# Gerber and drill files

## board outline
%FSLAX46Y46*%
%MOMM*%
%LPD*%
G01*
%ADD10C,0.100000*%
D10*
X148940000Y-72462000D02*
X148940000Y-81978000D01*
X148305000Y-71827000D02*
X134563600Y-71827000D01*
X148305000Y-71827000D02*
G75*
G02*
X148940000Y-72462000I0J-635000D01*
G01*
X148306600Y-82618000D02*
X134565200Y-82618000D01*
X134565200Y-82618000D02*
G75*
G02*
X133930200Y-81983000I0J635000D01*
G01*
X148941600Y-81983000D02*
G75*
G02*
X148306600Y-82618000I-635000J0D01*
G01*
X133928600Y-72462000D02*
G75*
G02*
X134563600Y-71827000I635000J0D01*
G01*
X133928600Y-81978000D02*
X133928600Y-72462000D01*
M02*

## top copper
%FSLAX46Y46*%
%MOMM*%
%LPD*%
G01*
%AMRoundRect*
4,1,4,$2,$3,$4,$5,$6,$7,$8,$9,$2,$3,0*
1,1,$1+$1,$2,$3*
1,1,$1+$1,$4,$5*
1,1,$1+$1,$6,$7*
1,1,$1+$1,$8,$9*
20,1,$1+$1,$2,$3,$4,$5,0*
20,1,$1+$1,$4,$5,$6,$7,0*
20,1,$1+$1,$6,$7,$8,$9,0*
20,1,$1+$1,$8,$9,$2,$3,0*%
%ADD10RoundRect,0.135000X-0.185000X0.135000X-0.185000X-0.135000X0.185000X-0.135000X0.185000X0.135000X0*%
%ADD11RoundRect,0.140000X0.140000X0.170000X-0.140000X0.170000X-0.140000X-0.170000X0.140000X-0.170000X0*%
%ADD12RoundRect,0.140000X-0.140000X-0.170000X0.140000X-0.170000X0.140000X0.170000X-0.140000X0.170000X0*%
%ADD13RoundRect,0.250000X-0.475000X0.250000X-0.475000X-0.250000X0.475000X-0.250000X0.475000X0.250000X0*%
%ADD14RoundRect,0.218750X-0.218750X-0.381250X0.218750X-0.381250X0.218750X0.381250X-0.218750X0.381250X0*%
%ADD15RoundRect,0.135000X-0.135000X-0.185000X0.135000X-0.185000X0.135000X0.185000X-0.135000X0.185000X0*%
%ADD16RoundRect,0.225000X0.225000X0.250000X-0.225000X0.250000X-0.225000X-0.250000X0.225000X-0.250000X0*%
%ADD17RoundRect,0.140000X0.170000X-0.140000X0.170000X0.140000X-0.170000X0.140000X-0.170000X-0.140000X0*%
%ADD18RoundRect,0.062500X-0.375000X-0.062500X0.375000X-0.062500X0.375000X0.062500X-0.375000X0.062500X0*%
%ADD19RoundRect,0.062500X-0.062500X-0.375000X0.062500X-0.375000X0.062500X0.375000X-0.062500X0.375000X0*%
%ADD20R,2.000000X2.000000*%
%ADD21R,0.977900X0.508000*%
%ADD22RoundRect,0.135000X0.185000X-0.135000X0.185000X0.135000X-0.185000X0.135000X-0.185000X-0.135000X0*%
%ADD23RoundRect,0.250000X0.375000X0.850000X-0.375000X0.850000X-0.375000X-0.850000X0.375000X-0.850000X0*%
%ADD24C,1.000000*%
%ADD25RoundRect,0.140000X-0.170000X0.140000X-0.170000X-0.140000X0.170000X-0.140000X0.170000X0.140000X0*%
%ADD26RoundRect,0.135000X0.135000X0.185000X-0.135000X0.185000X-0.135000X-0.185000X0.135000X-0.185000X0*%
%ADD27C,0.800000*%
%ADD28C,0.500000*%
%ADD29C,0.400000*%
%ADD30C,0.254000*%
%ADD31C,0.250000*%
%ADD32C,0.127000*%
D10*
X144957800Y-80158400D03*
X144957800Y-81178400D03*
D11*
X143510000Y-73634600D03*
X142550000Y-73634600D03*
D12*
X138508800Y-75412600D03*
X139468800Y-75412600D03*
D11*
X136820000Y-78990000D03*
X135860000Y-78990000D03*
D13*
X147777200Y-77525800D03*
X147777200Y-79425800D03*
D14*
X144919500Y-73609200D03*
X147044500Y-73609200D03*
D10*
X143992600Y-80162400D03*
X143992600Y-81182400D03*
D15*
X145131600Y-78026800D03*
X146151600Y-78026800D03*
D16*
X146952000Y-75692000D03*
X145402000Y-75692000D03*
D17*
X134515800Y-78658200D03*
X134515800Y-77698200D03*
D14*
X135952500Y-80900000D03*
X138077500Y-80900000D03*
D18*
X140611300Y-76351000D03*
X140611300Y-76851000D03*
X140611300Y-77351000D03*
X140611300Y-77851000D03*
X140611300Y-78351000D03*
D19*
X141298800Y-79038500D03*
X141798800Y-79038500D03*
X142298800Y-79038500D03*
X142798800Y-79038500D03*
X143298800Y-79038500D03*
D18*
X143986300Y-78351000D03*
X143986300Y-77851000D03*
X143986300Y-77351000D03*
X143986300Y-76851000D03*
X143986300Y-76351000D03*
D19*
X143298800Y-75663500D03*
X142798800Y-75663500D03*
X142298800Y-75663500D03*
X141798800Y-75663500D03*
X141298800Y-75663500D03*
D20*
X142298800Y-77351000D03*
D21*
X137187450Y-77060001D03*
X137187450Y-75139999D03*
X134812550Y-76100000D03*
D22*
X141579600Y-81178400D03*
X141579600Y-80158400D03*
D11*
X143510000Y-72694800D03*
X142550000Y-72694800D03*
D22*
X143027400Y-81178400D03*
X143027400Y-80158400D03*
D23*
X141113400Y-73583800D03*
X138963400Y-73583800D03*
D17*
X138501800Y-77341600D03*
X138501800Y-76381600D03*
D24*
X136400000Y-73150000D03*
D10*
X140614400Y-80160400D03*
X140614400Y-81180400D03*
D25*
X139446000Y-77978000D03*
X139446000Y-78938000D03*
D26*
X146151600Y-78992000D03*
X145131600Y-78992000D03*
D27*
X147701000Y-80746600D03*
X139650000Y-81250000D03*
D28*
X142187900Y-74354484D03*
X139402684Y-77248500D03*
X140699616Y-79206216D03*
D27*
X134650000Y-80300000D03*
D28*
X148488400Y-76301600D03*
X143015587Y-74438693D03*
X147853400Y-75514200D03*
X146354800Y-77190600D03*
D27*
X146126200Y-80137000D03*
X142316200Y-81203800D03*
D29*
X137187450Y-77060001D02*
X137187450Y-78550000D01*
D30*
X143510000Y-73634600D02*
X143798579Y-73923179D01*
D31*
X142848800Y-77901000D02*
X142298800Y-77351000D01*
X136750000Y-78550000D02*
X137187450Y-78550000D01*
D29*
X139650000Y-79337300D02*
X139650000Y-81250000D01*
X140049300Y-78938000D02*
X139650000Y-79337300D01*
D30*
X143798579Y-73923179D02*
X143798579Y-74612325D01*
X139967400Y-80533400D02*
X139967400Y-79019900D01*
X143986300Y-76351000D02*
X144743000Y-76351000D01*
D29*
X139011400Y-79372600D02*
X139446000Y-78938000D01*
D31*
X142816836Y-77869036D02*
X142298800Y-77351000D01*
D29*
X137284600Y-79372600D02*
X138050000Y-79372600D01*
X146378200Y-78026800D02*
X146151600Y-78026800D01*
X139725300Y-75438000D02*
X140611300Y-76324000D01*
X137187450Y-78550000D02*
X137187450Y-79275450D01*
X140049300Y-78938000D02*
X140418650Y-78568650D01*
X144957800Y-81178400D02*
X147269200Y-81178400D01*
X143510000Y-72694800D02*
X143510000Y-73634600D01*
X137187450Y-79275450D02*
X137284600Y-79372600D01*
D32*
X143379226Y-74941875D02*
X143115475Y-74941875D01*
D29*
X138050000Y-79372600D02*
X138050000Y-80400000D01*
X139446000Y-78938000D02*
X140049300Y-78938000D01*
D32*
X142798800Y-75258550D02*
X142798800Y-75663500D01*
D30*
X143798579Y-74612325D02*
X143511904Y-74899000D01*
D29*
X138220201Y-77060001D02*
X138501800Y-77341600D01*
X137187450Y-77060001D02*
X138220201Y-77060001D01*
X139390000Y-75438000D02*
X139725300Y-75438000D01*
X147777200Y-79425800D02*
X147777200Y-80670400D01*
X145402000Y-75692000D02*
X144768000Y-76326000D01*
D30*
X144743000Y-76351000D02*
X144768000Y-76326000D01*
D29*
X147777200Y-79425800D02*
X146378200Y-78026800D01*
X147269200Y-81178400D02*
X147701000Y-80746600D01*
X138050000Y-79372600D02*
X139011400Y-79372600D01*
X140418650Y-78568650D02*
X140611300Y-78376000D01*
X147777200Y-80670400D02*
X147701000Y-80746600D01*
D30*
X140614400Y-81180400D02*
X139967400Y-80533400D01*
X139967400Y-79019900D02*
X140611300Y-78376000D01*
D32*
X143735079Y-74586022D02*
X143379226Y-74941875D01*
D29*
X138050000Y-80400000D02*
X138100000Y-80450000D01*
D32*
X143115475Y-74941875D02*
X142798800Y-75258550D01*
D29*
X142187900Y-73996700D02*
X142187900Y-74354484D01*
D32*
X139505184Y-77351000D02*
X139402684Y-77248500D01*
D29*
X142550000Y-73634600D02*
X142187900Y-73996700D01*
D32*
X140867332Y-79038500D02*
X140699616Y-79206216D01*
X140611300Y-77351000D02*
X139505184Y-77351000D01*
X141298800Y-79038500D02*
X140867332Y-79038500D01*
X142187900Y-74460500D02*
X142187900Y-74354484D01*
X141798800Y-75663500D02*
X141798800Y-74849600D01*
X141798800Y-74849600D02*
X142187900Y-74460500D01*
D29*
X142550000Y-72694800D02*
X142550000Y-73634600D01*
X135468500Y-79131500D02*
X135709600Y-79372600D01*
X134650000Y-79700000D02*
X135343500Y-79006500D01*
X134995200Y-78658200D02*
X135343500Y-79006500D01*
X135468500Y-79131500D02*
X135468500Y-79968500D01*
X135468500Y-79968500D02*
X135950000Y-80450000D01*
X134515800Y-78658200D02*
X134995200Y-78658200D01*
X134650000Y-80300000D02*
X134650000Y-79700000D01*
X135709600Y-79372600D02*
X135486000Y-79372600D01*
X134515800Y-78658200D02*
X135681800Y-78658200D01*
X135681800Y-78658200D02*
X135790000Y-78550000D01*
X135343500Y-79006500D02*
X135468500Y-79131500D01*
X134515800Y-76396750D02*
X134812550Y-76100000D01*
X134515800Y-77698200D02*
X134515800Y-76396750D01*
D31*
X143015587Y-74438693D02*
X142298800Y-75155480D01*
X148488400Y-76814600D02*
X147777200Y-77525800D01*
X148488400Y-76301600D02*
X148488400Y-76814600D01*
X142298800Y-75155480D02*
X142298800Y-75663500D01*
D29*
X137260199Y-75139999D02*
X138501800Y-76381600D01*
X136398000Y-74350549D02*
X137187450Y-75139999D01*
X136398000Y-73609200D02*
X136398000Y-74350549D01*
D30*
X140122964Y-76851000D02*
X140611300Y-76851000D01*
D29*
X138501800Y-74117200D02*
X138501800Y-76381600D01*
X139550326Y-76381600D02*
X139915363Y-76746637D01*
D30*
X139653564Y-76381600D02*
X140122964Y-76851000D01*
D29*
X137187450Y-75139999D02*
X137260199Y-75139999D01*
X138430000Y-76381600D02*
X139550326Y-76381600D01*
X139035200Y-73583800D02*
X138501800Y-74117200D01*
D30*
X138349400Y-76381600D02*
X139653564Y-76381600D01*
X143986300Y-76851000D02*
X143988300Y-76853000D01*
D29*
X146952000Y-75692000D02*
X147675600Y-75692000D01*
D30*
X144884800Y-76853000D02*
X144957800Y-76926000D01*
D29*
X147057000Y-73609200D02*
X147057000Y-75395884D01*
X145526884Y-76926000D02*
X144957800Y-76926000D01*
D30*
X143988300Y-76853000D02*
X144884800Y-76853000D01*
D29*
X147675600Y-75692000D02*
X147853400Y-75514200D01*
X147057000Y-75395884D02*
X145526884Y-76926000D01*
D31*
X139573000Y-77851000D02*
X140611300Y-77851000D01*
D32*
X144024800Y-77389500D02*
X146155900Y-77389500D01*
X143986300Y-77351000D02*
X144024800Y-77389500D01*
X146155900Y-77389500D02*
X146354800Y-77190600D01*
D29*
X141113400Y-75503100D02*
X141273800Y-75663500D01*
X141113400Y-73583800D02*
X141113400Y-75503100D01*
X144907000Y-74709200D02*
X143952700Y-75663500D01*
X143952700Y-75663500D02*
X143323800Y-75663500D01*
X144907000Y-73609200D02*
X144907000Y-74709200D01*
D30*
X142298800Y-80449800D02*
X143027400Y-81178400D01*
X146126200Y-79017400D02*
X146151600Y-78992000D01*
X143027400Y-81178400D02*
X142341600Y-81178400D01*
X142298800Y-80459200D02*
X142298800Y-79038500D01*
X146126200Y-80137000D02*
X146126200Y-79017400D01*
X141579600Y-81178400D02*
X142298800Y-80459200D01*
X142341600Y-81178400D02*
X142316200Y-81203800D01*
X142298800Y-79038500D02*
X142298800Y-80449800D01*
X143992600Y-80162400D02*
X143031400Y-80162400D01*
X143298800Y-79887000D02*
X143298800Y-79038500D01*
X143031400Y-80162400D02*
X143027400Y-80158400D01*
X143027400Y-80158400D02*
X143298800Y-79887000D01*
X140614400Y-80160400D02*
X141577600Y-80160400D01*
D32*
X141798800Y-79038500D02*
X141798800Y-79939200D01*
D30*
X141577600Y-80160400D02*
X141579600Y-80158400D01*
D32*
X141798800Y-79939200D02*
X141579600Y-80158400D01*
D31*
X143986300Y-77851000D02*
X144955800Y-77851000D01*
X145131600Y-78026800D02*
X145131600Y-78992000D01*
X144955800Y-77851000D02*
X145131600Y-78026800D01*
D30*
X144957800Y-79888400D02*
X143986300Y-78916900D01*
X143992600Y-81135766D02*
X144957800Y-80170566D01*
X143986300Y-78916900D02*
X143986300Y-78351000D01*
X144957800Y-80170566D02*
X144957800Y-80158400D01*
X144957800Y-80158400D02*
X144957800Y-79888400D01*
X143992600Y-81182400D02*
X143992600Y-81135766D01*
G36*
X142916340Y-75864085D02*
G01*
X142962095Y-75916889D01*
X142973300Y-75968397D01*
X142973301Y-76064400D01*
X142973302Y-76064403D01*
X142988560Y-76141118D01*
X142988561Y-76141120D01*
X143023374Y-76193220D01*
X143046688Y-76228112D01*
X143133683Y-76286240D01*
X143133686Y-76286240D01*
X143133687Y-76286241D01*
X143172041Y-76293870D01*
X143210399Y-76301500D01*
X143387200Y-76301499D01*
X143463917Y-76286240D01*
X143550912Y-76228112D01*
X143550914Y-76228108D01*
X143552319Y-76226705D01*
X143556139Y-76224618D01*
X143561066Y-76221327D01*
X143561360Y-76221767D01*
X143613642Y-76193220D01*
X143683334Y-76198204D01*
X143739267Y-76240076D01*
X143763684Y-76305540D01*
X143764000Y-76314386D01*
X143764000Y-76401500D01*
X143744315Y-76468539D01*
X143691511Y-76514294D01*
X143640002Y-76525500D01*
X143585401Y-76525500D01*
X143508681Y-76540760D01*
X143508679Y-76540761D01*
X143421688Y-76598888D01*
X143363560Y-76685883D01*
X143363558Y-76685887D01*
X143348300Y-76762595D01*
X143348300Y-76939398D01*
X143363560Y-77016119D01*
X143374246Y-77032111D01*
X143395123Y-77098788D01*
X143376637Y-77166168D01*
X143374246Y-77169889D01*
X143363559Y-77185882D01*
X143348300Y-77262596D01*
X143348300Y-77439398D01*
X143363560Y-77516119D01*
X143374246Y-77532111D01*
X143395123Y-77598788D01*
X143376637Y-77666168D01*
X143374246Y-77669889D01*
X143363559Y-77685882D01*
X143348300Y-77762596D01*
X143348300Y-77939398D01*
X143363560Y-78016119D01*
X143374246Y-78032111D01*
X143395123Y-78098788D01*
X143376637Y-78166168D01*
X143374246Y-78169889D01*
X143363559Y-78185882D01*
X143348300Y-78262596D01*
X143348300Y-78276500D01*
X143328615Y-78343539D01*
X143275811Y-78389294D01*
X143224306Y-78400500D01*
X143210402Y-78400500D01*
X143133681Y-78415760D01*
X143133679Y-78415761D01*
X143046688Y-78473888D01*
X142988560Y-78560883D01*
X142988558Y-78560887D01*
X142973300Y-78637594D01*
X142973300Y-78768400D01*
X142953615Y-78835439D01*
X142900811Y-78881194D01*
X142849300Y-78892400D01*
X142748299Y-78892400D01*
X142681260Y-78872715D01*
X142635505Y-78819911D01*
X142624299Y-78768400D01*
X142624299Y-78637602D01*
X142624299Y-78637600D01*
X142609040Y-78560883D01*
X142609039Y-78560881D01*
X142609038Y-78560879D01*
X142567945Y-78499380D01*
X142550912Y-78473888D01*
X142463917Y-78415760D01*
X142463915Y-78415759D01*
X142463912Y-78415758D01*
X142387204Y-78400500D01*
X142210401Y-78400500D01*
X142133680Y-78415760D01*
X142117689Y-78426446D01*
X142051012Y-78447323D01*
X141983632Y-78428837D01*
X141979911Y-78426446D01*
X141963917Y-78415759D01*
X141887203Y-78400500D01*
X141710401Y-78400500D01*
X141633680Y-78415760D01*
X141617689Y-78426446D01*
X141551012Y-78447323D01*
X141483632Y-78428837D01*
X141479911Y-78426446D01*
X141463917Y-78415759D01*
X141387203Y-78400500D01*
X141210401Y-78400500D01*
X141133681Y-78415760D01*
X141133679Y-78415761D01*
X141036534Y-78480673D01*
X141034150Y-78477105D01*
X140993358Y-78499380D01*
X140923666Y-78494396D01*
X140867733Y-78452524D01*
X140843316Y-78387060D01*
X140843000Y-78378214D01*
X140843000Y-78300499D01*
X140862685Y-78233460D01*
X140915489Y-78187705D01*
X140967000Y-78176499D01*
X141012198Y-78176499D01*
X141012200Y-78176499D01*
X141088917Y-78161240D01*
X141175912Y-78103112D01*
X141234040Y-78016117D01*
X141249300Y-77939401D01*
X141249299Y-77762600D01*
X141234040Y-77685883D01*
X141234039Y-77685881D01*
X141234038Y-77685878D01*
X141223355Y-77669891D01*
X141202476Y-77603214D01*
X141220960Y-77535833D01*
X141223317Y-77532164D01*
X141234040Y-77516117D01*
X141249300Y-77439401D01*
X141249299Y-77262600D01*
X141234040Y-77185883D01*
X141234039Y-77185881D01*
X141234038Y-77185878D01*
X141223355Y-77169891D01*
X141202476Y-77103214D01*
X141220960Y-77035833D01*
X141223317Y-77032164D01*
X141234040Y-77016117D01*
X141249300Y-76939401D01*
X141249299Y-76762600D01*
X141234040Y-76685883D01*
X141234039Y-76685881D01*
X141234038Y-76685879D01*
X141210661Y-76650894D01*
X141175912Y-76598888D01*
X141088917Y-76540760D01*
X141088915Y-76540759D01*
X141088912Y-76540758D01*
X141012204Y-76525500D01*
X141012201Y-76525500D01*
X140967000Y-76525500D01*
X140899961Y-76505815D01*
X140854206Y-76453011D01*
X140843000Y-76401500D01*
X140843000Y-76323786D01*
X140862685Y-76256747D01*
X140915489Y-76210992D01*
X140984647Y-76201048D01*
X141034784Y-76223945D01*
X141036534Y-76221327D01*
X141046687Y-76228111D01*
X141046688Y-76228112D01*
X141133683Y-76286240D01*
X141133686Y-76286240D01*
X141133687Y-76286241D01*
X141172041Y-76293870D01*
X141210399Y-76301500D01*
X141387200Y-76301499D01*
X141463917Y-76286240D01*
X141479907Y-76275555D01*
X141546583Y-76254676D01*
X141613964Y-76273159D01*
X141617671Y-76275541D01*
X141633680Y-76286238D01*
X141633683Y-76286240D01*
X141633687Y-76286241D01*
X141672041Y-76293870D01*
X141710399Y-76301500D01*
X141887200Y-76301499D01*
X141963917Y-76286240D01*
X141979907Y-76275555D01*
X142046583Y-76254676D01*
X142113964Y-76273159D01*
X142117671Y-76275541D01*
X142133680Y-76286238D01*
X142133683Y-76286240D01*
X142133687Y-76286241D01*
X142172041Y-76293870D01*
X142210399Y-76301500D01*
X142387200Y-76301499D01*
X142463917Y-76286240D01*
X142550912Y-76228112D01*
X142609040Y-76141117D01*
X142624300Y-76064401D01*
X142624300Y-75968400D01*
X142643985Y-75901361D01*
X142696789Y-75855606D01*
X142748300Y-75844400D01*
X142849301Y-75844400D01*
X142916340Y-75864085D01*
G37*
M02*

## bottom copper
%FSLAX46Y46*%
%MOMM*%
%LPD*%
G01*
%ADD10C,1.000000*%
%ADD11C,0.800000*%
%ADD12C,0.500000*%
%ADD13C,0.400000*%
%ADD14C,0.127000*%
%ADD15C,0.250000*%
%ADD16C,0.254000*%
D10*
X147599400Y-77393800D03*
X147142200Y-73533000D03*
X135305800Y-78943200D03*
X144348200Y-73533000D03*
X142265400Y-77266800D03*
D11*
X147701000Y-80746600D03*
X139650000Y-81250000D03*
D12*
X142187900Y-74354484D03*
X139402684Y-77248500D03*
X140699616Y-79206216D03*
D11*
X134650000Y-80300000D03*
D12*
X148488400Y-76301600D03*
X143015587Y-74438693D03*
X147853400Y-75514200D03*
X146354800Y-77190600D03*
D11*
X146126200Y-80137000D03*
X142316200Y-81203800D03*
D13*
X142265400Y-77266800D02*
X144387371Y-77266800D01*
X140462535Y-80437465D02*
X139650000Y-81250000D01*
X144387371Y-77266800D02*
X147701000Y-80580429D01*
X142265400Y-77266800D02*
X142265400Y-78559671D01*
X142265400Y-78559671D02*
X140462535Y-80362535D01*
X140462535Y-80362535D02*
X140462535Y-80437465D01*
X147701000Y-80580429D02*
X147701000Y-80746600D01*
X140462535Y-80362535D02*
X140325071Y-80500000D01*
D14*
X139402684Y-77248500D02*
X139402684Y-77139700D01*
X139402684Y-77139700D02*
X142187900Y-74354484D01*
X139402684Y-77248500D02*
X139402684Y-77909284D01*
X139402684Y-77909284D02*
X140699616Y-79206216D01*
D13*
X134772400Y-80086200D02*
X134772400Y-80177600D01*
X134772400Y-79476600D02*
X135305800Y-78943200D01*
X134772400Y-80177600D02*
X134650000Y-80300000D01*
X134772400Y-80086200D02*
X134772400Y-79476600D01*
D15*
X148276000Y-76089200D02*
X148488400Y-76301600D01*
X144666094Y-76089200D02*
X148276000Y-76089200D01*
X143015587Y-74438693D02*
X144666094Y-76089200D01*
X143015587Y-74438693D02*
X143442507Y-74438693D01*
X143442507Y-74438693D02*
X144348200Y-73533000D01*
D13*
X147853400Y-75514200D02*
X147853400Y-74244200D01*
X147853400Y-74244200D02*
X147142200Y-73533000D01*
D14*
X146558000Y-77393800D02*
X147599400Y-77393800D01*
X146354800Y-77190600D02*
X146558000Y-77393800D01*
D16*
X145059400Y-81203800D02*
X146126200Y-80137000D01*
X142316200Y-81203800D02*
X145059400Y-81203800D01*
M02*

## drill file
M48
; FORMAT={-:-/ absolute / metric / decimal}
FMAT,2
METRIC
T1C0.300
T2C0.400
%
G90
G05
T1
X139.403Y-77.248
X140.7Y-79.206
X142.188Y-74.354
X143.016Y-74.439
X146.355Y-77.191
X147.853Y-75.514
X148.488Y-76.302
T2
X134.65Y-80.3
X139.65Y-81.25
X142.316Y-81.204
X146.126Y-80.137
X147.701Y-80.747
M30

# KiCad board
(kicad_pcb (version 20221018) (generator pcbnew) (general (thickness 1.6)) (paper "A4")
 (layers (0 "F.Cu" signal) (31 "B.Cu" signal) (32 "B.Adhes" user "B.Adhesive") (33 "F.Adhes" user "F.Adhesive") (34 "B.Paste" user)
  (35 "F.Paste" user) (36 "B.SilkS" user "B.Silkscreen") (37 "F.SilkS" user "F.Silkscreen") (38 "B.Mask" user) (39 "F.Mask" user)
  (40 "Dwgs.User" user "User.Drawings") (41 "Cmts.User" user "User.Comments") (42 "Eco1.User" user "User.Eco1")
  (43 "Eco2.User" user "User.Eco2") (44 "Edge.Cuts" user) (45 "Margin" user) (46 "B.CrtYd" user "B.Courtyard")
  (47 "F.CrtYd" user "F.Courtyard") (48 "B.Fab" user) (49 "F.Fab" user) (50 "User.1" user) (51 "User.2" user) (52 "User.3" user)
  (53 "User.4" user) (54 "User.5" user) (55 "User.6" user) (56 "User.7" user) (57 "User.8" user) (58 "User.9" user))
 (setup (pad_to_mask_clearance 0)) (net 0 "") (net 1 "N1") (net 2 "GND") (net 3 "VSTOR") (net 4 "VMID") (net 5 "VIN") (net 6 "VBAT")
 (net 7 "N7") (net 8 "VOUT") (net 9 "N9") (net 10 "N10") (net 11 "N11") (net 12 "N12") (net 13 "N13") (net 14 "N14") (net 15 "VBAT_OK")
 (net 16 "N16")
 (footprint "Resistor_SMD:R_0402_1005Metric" (layer "F.Cu") (at 144.9578 80.6684 -90)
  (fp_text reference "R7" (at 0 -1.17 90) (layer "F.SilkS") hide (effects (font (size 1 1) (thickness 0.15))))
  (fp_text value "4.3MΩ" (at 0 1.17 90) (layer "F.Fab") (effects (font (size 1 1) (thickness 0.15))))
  (pad "1" smd roundrect (at -0.51 0 270) (size 0.54 0.64) (layers "F.Cu" "F.Paste" "F.Mask") (roundrect_rratio 0.25) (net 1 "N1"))
  (pad "2" smd roundrect (at 0.51 0 270) (size 0.54 0.64) (layers "F.Cu" "F.Paste" "F.Mask") (roundrect_rratio 0.25) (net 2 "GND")))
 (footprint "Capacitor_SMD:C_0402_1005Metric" (layer "F.Cu") (at 143.03 73.6346 180)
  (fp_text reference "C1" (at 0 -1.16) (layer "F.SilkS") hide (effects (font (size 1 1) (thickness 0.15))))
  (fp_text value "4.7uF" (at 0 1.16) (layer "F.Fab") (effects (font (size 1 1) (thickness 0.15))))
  (pad "1" smd roundrect (at -0.48 0 180) (size 0.56 0.62) (layers "F.Cu" "F.Paste" "F.Mask") (roundrect_rratio 0.25) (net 2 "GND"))
  (pad "2" smd roundrect (at 0.48 0 180) (size 0.56 0.62) (layers "F.Cu" "F.Paste" "F.Mask") (roundrect_rratio 0.25) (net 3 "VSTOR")))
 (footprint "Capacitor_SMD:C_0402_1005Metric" (layer "F.Cu") (at 138.9888 75.4126)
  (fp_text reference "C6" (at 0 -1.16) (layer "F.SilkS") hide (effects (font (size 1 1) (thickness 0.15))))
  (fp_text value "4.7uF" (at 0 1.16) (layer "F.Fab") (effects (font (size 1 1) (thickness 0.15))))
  (pad "1" smd roundrect (at -0.48 0) (size 0.56 0.62) (layers "F.Cu" "F.Paste" "F.Mask") (roundrect_rratio 0.25) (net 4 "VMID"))
  (pad "2" smd roundrect (at 0.48 0) (size 0.56 0.62) (layers "F.Cu" "F.Paste" "F.Mask") (roundrect_rratio 0.25) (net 2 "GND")))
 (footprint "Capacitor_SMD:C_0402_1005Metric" (layer "F.Cu") (at 136.34 78.99 180)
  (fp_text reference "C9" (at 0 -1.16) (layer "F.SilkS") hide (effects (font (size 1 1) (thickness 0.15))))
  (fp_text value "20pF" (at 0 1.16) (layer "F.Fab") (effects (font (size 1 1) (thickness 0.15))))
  (pad "1" smd roundrect (at -0.48 0 180) (size 0.56 0.62) (layers "F.Cu" "F.Paste" "F.Mask") (roundrect_rratio 0.25) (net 2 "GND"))
  (pad "2" smd roundrect (at 0.48 0 180) (size 0.56 0.62) (layers "F.Cu" "F.Paste" "F.Mask") (roundrect_rratio 0.25) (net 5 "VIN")))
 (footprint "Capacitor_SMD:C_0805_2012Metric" (layer "F.Cu") (at 147.7772 78.4758 -90)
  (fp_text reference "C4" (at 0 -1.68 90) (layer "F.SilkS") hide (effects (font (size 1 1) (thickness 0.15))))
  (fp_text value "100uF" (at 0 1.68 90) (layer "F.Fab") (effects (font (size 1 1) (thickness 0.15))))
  (pad "1" smd roundrect (at -0.95 0 270) (size 1 1.45) (layers "F.Cu" "F.Paste" "F.Mask") (roundrect_rratio 0.25) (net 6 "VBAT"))
  (pad "2" smd roundrect (at 0.95 0 270) (size 1 1.45) (layers "F.Cu" "F.Paste" "F.Mask") (roundrect_rratio 0.25) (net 2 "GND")))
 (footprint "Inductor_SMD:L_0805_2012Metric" (layer "F.Cu") (at 145.982 73.6092)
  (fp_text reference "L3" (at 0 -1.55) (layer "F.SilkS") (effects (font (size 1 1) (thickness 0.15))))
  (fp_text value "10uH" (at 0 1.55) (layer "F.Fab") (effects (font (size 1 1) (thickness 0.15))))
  (pad "1" smd roundrect (at -1.0625 0) (size 0.875 1.2) (layers "F.Cu" "F.Paste" "F.Mask") (roundrect_rratio 0.25) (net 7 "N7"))
  (pad "2" smd roundrect (at 1.0625 0) (size 0.875 1.2) (layers "F.Cu" "F.Paste" "F.Mask") (roundrect_rratio 0.25) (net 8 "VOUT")))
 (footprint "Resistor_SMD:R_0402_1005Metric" (layer "F.Cu") (at 143.9926 80.6724 -90)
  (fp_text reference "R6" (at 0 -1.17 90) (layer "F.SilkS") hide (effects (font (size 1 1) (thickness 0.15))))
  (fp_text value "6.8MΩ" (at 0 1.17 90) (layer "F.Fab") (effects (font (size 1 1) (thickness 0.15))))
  (pad "1" smd roundrect (at -0.51 0 270) (size 0.54 0.64) (layers "F.Cu" "F.Paste" "F.Mask") (roundrect_rratio 0.25) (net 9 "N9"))
  (pad "2" smd roundrect (at 0.51 0 270) (size 0.54 0.64) (layers "F.Cu" "F.Paste" "F.Mask") (roundrect_rratio 0.25) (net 1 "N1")))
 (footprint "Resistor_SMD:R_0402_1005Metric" (layer "F.Cu") (at 145.6416 78.0268)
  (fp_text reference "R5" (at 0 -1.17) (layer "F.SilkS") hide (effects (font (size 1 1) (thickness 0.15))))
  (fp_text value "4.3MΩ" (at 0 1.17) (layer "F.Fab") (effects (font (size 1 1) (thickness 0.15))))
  (pad "1" smd roundrect (at -0.51 0) (size 0.54 0.64) (layers "F.Cu" "F.Paste" "F.Mask") (roundrect_rratio 0.25) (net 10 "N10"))
  (pad "2" smd roundrect (at 0.51 0) (size 0.54 0.64) (layers "F.Cu" "F.Paste" "F.Mask") (roundrect_rratio 0.25) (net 2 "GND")))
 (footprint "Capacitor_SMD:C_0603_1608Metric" (layer "F.Cu") (at 146.177 75.692 180)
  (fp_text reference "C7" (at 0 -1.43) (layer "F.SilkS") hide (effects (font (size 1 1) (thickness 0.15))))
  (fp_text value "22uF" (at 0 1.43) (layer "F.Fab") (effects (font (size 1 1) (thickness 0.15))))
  (pad "1" smd roundrect (at -0.775 0 180) (size 0.9 0.95) (layers "F.Cu" "F.Paste" "F.Mask") (roundrect_rratio 0.25) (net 8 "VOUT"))
  (pad "2" smd roundrect (at 0.775 0 180) (size 0.9 0.95) (layers "F.Cu" "F.Paste" "F.Mask") (roundrect_rratio 0.25) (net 2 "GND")))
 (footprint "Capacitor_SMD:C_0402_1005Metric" (layer "F.Cu") (at 134.5158 78.1782 90)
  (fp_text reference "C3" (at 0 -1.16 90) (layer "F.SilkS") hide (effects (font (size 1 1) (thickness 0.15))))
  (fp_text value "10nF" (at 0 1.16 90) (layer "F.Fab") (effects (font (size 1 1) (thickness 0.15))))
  (pad "1" smd roundrect (at -0.48 0 90) (size 0.56 0.62) (layers "F.Cu" "F.Paste" "F.Mask") (roundrect_rratio 0.25) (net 5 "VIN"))
  (pad "2" smd roundrect (at 0.48 0 90) (size 0.56 0.62) (layers "F.Cu" "F.Paste" "F.Mask") (roundrect_rratio 0.25) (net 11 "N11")))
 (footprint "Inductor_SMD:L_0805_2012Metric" (layer "F.Cu") (at 137.015 80.9)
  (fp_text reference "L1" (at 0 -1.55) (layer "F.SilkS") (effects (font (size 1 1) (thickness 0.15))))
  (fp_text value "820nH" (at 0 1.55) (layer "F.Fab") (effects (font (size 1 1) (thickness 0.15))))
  (pad "1" smd roundrect (at -1.0625 0) (size 0.875 1.2) (layers "F.Cu" "F.Paste" "F.Mask") (roundrect_rratio 0.25) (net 5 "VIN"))
  (pad "2" smd roundrect (at 1.0625 0) (size 0.875 1.2) (layers "F.Cu" "F.Paste" "F.Mask") (roundrect_rratio 0.25) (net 2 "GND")))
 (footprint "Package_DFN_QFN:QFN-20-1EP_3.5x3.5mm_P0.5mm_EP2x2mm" (layer "F.Cu") (at 142.2988 77.351)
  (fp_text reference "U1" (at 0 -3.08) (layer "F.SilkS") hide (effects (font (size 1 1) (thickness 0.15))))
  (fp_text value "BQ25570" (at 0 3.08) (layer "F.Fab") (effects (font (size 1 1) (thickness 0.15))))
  (pad "" smd roundrect (at -0.5 -0.5) (size 0.81 0.81) (layers "F.Paste") (roundrect_rratio 0.25))
  (pad "" smd roundrect (at -0.5 0.5) (size 0.81 0.81) (layers "F.Paste") (roundrect_rratio 0.25))
  (pad "" smd roundrect (at 0.5 -0.5) (size 0.81 0.81) (layers "F.Paste") (roundrect_rratio 0.25))
  (pad "" smd roundrect (at 0.5 0.5) (size 0.81 0.81) (layers "F.Paste") (roundrect_rratio 0.25))
  (pad "1" smd roundrect (at -1.6875 -1) (size 0.875 0.25) (layers "F.Cu" "F.Paste" "F.Mask") (roundrect_rratio 0.25) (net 2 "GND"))
  (pad "2" smd roundrect (at -1.6875 -0.5) (size 0.875 0.25) (layers "F.Cu" "F.Paste" "F.Mask") (roundrect_rratio 0.25) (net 4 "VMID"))
  (pad "3" smd roundrect (at -1.6875 0) (size 0.875 0.25) (layers "F.Cu" "F.Paste" "F.Mask") (roundrect_rratio 0.25) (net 3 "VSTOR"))
  (pad "4" smd roundrect (at -1.6875 0.5) (size 0.875 0.25) (layers "F.Cu" "F.Paste" "F.Mask") (roundrect_rratio 0.25) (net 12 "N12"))
  (pad "5" smd roundrect (at -1.6875 1) (size 0.875 0.25) (layers "F.Cu" "F.Paste" "F.Mask") (roundrect_rratio 0.25) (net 2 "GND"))
  (pad "6" smd roundrect (at -1 1.6875) (size 0.25 0.875) (layers "F.Cu" "F.Paste" "F.Mask") (roundrect_rratio 0.25) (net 3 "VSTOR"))
  (pad "7" smd roundrect (at -0.5 1.6875) (size 0.25 0.875) (layers "F.Cu" "F.Paste" "F.Mask") (roundrect_rratio 0.25) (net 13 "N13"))
  (pad "8" smd roundrect (at 0 1.6875) (size 0.25 0.875) (layers "F.Cu" "F.Paste" "F.Mask") (roundrect_rratio 0.25) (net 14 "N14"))
  (pad "9" smd roundrect (at 0.5 1.6875) (size 0.25 0.875) (layers "F.Cu" "F.Paste" "F.Mask") (roundrect_rratio 0.25) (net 2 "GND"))
  (pad "10" smd roundrect (at 1 1.6875) (size 0.25 0.875) (layers "F.Cu" "F.Paste" "F.Mask") (roundrect_rratio 0.25) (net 9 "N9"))
  (pad "11" smd roundrect (at 1.6875 1) (size 0.875 0.25) (layers "F.Cu" "F.Paste" "F.Mask") (roundrect_rratio 0.25) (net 1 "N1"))
  (pad "12" smd roundrect (at 1.6875 0.5) (size 0.875 0.25) (layers "F.Cu" "F.Paste" "F.Mask") (roundrect_rratio 0.25) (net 10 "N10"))
  (pad "13" smd roundrect (at 1.6875 0) (size 0.875 0.25) (layers "F.Cu" "F.Paste" "F.Mask") (roundrect_rratio 0.25) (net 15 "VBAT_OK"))
  (pad "14" smd roundrect (at 1.6875 -0.5) (size 0.875 0.25) (layers "F.Cu" "F.Paste" "F.Mask") (roundrect_rratio 0.25) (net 8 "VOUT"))
  (pad "15" smd roundrect (at 1.6875 -1) (size 0.875 0.25) (layers "F.Cu" "F.Paste" "F.Mask") (roundrect_rratio 0.25) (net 2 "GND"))
  (pad "16" smd roundrect (at 1 -1.6875) (size 0.25 0.875) (layers "F.Cu" "F.Paste" "F.Mask") (roundrect_rratio 0.25) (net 7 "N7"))
  (pad "17" smd roundrect (at 0.5 -1.6875) (size 0.25 0.875) (layers "F.Cu" "F.Paste" "F.Mask") (roundrect_rratio 0.25) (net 2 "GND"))
  (pad "18" smd roundrect (at 0 -1.6875) (size 0.25 0.875) (layers "F.Cu" "F.Paste" "F.Mask") (roundrect_rratio 0.25) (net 6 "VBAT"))
  (pad "19" smd roundrect (at -0.5 -1.6875) (size 0.25 0.875) (layers "F.Cu" "F.Paste" "F.Mask") (roundrect_rratio 0.25) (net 3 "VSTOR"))
  (pad "20" smd roundrect (at -1 -1.6875) (size 0.25 0.875) (layers "F.Cu" "F.Paste" "F.Mask") (roundrect_rratio 0.25) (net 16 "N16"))
  (pad "21" smd rect (at 0 0) (size 2 2) (layers "F.Cu" "F.Mask") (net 2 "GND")))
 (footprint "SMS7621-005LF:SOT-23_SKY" (layer "F.Cu") (at 136 76.1 180)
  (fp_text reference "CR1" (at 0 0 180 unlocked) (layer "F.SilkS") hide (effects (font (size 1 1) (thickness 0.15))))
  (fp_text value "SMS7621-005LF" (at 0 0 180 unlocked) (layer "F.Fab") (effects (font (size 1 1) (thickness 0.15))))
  (pad "1" smd rect (at -1.18745 -0.960001 180) (size 0.9779 0.508) (layers "F.Cu" "F.Paste" "F.Mask") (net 2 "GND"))
  (pad "2" smd rect (at -1.18745 0.960001 180) (size 0.9779 0.508) (layers "F.Cu" "F.Paste" "F.Mask") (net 4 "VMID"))
  (pad "3" smd rect (at 1.18745 0 180) (size 0.9779 0.508) (layers "F.Cu" "F.Paste" "F.Mask") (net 11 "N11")))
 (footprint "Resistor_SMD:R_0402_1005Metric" (layer "F.Cu") (at 141.5796 80.6684 90)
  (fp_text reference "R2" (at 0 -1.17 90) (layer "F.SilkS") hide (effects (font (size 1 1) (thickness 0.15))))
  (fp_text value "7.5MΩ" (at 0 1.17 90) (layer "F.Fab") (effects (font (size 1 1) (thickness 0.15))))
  (pad "1" smd roundrect (at -0.51 0 90) (size 0.54 0.64) (layers "F.Cu" "F.Paste" "F.Mask") (roundrect_rratio 0.25) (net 14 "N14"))
  (pad "2" smd roundrect (at 0.51 0 90) (size 0.54 0.64) (layers "F.Cu" "F.Paste" "F.Mask") (roundrect_rratio 0.25) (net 13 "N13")))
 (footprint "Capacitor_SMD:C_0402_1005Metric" (layer "F.Cu") (at 143.03 72.6948 180)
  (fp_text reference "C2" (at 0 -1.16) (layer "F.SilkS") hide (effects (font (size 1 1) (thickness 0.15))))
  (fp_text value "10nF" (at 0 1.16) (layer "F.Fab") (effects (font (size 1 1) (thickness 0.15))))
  (pad "1" smd roundrect (at -0.48 0 180) (size 0.56 0.62) (layers "F.Cu" "F.Paste" "F.Mask") (roundrect_rratio 0.25) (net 2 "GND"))
  (pad "2" smd roundrect (at 0.48 0 180) (size 0.56 0.62) (layers "F.Cu" "F.Paste" "F.Mask") (roundrect_rratio 0.25) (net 3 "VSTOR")))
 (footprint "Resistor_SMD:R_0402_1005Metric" (layer "F.Cu") (at 143.0274 80.6684 90)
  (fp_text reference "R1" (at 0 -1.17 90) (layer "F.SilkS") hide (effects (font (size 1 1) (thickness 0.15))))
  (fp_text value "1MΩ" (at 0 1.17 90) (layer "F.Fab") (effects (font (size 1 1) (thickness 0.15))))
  (pad "1" smd roundrect (at -0.51 0 90) (size 0.54 0.64) (layers "F.Cu" "F.Paste" "F.Mask") (roundrect_rratio 0.25) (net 14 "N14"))
  (pad "2" smd roundrect (at 0.51 0 90) (size 0.54 0.64) (layers "F.Cu" "F.Paste" "F.Mask") (roundrect_rratio 0.25) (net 9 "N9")))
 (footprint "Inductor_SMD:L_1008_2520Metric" (layer "F.Cu") (at 140.0384 73.5838 180)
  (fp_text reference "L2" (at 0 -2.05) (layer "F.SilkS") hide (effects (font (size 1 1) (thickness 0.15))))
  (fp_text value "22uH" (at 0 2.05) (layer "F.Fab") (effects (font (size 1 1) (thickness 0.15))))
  (pad "1" smd roundrect (at -1.075 0 180) (size 1.25 2.2) (layers "F.Cu" "F.Paste" "F.Mask") (roundrect_rratio 0.2) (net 16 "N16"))
  (pad "2" smd roundrect (at 1.075 0 180) (size 1.25 2.2) (layers "F.Cu" "F.Paste" "F.Mask") (roundrect_rratio 0.2) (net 4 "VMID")))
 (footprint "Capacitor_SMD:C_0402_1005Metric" (layer "F.Cu") (at 138.5018 76.8616 90)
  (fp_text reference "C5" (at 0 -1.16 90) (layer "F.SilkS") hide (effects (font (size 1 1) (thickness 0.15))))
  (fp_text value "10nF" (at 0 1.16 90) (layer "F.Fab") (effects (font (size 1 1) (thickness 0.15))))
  (pad "1" smd roundrect (at -0.48 0 90) (size 0.56 0.62) (layers "F.Cu" "F.Paste" "F.Mask") (roundrect_rratio 0.25) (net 2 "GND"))
  (pad "2" smd roundrect (at 0.48 0 90) (size 0.56 0.62) (layers "F.Cu" "F.Paste" "F.Mask") (roundrect_rratio 0.25) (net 4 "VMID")))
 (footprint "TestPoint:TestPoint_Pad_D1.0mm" (layer "F.Cu") (at 136.4 73.15)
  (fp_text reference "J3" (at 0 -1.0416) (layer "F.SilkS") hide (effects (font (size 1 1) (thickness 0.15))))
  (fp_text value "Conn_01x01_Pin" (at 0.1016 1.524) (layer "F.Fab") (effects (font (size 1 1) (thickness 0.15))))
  (pad "1" smd circle (at 0 0) (size 1 1) (layers "F.Cu" "F.Mask") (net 4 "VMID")))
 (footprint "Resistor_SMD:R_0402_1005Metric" (layer "F.Cu") (at 140.6144 80.6704 -90)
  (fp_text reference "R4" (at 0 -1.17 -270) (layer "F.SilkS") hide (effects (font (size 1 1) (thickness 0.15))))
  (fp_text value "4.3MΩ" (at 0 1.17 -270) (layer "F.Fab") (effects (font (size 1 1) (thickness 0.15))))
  (pad "1" smd roundrect (at -0.51 0 270) (size 0.54 0.64) (layers "F.Cu" "F.Paste" "F.Mask") (roundrect_rratio 0.25) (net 13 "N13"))
  (pad "2" smd roundrect (at 0.51 0 270) (size 0.54 0.64) (layers "F.Cu" "F.Paste" "F.Mask") (roundrect_rratio 0.25) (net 2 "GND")))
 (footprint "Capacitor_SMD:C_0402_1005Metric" (layer "F.Cu") (at 139.446 78.458 -90)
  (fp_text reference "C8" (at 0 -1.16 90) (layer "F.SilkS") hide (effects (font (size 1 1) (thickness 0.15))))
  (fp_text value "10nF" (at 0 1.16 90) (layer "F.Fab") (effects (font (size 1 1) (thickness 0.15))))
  (pad "1" smd roundrect (at -0.48 0 270) (size 0.56 0.62) (layers "F.Cu" "F.Paste" "F.Mask") (roundrect_rratio 0.25) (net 12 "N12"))
  (pad "2" smd roundrect (at 0.48 0 270) (size 0.56 0.62) (layers "F.Cu" "F.Paste" "F.Mask") (roundrect_rratio 0.25) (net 2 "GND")))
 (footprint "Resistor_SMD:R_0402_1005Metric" (layer "F.Cu") (at 145.6416 78.992 180)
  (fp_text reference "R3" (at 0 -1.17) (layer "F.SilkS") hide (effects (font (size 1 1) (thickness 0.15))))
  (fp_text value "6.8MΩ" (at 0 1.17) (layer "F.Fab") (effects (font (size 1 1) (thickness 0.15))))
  (pad "1" smd roundrect (at -0.51 0 180) (size 0.54 0.64) (layers "F.Cu" "F.Paste" "F.Mask") (roundrect_rratio 0.25) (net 14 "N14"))
  (pad "2" smd roundrect (at 0.51 0 180) (size 0.54 0.64) (layers "F.Cu" "F.Paste" "F.Mask") (roundrect_rratio 0.25) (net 10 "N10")))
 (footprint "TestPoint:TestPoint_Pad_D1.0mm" (layer "B.Cu") (at 147.5994 77.3938 180)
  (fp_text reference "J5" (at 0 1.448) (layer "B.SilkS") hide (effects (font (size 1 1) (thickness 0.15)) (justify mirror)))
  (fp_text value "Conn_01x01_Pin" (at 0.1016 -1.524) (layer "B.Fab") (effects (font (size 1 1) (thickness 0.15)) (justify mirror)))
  (pad "1" smd circle (at 0 0 180) (size 1 1) (layers "B.Cu" "B.Mask") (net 15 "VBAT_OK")))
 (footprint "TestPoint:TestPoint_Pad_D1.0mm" (layer "B.Cu") (at 147.1422 73.533 180)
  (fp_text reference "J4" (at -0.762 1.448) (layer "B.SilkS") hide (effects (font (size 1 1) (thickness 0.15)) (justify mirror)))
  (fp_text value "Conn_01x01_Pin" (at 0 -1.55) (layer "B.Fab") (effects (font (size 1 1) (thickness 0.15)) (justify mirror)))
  (pad "1" smd circle (at 0 0 180) (size 1 1) (layers "B.Cu" "B.Mask") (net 8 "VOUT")))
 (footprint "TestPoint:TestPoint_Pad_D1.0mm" (layer "B.Cu") (at 135.3058 78.9432 180)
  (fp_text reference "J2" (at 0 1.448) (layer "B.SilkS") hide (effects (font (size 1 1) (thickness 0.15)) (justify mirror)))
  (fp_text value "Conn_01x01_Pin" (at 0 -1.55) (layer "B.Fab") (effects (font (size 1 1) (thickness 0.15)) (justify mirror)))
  (pad "1" smd circle (at 0 0 180) (size 1 1) (layers "B.Cu" "B.Mask") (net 5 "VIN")))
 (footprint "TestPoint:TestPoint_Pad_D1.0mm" (layer "B.Cu") (at 144.3482 73.533 180)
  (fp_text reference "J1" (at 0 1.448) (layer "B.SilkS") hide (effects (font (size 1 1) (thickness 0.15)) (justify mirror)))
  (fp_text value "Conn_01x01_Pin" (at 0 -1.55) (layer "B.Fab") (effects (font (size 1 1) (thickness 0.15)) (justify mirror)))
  (pad "1" smd circle (at 0 0 180) (size 1 1) (layers "B.Cu" "B.Mask") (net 6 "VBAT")))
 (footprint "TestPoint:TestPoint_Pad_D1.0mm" (layer "B.Cu") (at 142.2654 77.2668 180)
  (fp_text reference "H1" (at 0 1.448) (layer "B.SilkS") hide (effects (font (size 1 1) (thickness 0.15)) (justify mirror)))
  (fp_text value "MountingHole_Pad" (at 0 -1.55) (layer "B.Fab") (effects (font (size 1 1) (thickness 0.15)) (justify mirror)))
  (pad "1" smd circle (at 0 0 180) (size 1 1) (layers "B.Cu" "B.Mask") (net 2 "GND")))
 (gr_line (start 148.94 72.462) (end 148.94 81.978) (stroke (width 0.1) (type default)) (layer "Edge.Cuts"))
 (gr_line (start 148.305 71.827) (end 134.5636 71.827) (stroke (width 0.1) (type default)) (layer "Edge.Cuts"))
 (gr_arc (start 148.305 71.827) (mid 148.754013 72.012987) (end 148.94 72.462) (stroke (width 0.1) (type default)) (layer "Edge.Cuts"))
 (gr_line (start 148.3066 82.618) (end 134.5652 82.618) (stroke (width 0.1) (type default)) (layer "Edge.Cuts"))
 (gr_arc (start 134.5652 82.618) (mid 134.116187 82.432013) (end 133.9302 81.983) (stroke (width 0.1) (type default)) (layer "Edge.Cuts"))
 (gr_arc (start 148.9416 81.983) (mid 148.755613 82.432013) (end 148.3066 82.618) (stroke (width 0.1) (type default)) (layer "Edge.Cuts"))
 (gr_arc (start 133.9286 72.462) (mid 134.114587 72.012987) (end 134.5636 71.827) (stroke (width 0.1) (type default)) (layer "Edge.Cuts"))
 (gr_line (start 133.9286 81.978) (end 133.9286 72.462) (stroke (width 0.1) (type default)) (layer "Edge.Cuts"))
 (segment (start 137.18745 77.060001) (end 137.18745 78.55) (width 0.4) (layer "F.Cu") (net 2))
 (segment (start 143.51 73.6346) (end 143.798579 73.923179) (width 0.254) (layer "F.Cu") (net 2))
 (segment (start 142.8488 77.901) (end 142.2988 77.351) (width 0.25) (layer "F.Cu") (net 2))
 (segment (start 136.75 78.55) (end 137.18745 78.55) (width 0.25) (layer "F.Cu") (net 2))
 (segment (start 139.65 79.3373) (end 139.65 81.25) (width 0.4) (layer "F.Cu") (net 2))
 (segment (start 140.0493 78.938) (end 139.65 79.3373) (width 0.4) (layer "F.Cu") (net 2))
 (segment (start 143.798579 73.923179) (end 143.798579 74.612325) (width 0.254) (layer "F.Cu") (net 2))
 (segment (start 139.9674 80.5334) (end 139.9674 79.0199) (width 0.254) (layer "F.Cu") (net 2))
 (segment (start 143.9863 76.351) (end 144.743 76.351) (width 0.254) (layer "F.Cu") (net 2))
 (segment (start 139.0114 79.3726) (end 139.446 78.938) (width 0.4) (layer "F.Cu") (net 2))
 (segment (start 142.816836 77.869036) (end 142.2988 77.351) (width 0.25) (layer "F.Cu") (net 2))
 (segment (start 137.2846 79.3726) (end 138.05 79.3726) (width 0.4) (layer "F.Cu") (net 2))
 (segment (start 146.3782 78.0268) (end 146.1516 78.0268) (width 0.4) (layer "F.Cu") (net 2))
 (segment (start 139.7253 75.438) (end 140.6113 76.324) (width 0.4) (layer "F.Cu") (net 2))
 (segment (start 137.18745 78.55) (end 137.18745 79.27545) (width 0.4) (layer "F.Cu") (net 2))
 (segment (start 140.0493 78.938) (end 140.41865 78.56865) (width 0.4) (layer "F.Cu") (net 2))
 (segment (start 144.9578 81.1784) (end 147.2692 81.1784) (width 0.4) (layer "F.Cu") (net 2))
 (segment (start 143.51 72.6948) (end 143.51 73.6346) (width 0.4) (layer "F.Cu") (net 2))
 (segment (start 137.18745 79.27545) (end 137.2846 79.3726) (width 0.4) (layer "F.Cu") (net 2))
 (segment (start 143.379226 74.941875) (end 143.115475 74.941875) (width 0.127) (layer "F.Cu") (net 2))
 (segment (start 138.05 79.3726) (end 138.05 80.4) (width 0.4) (layer "F.Cu") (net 2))
 (segment (start 139.446 78.938) (end 140.0493 78.938) (width 0.4) (layer "F.Cu") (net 2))
 (segment (start 142.7988 75.25855) (end 142.7988 75.6635) (width 0.127) (layer "F.Cu") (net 2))
 (segment (start 143.798579 74.612325) (end 143.511904 74.899) (width 0.254) (layer "F.Cu") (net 2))
 (segment (start 138.220201 77.060001) (end 138.5018 77.3416) (width 0.4) (layer "F.Cu") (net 2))
 (segment (start 137.18745 77.060001) (end 138.220201 77.060001) (width 0.4) (layer "F.Cu") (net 2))
 (segment (start 139.39 75.438) (end 139.7253 75.438) (width 0.4) (layer "F.Cu") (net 2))
 (segment (start 147.7772 79.4258) (end 147.7772 80.6704) (width 0.4) (layer "F.Cu") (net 2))
 (segment (start 145.402 75.692) (end 144.768 76.326) (width 0.4) (layer "F.Cu") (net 2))
 (segment (start 144.743 76.351) (end 144.768 76.326) (width 0.254) (layer "F.Cu") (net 2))
 (segment (start 147.7772 79.4258) (end 146.3782 78.0268) (width 0.4) (layer "F.Cu") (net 2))
 (segment (start 147.2692 81.1784) (end 147.701 80.7466) (width 0.4) (layer "F.Cu") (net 2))
 (segment (start 138.05 79.3726) (end 139.0114 79.3726) (width 0.4) (layer "F.Cu") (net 2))
 (segment (start 140.41865 78.56865) (end 140.6113 78.376) (width 0.4) (layer "F.Cu") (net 2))
 (segment (start 147.7772 80.6704) (end 147.701 80.7466) (width 0.4) (layer "F.Cu") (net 2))
 (segment (start 140.6144 81.1804) (end 139.9674 80.5334) (width 0.254) (layer "F.Cu") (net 2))
 (segment (start 139.9674 79.0199) (end 140.6113 78.376) (width 0.254) (layer "F.Cu") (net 2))
 (segment (start 143.735079 74.586022) (end 143.379226 74.941875) (width 0.127) (layer "F.Cu") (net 2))
 (segment (start 138.05 80.4) (end 138.1 80.45) (width 0.4) (layer "F.Cu") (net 2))
 (segment (start 143.115475 74.941875) (end 142.7988 75.25855) (width 0.127) (layer "F.Cu") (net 2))
 (via (at 147.701 80.7466) (size 0.8) (drill 0.4) (layers "F.Cu" "B.Cu") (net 2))
 (via (at 139.65 81.25) (size 0.8) (drill 0.4) (layers "F.Cu" "B.Cu") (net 2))
 (segment (start 142.2654 77.2668) (end 144.387371 77.2668) (width 0.4) (layer "B.Cu") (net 2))
 (segment (start 140.462535 80.437465) (end 139.65 81.25) (width 0.4) (layer "B.Cu") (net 2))
 (segment (start 144.387371 77.2668) (end 147.701 80.580429) (width 0.4) (layer "B.Cu") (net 2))
 (segment (start 142.2654 77.2668) (end 142.2654 78.559671) (width 0.4) (layer "B.Cu") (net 2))
 (segment (start 142.2654 78.559671) (end 140.462535 80.362535) (width 0.4) (layer "B.Cu") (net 2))
 (segment (start 140.462535 80.362535) (end 140.462535 80.437465) (width 0.4) (layer "B.Cu") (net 2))
 (segment (start 147.701 80.580429) (end 147.701 80.7466) (width 0.4) (layer "B.Cu") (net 2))
 (segment (start 140.462535 80.362535) (end 140.325071 80.5) (width 0.4) (layer "B.Cu") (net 2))
 (segment (start 142.1879 73.9967) (end 142.1879 74.354484) (width 0.4) (layer "F.Cu") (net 3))
 (segment (start 139.505184 77.351) (end 139.402684 77.2485) (width 0.127) (layer "F.Cu") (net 3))
 (segment (start 142.55 73.6346) (end 142.1879 73.9967) (width 0.4) (layer "F.Cu") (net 3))
 (segment (start 140.867332 79.0385) (end 140.699616 79.206216) (width 0.127) (layer "F.Cu") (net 3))
 (segment (start 140.6113 77.351) (end 139.505184 77.351) (width 0.127) (layer "F.Cu") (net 3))
 (segment (start 141.2988 79.0385) (end 140.867332 79.0385) (width 0.127) (layer "F.Cu") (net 3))
 (segment (start 142.1879 74.4605) (end 142.1879 74.354484) (width 0.127) (layer "F.Cu") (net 3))
 (segment (start 141.7988 75.6635) (end 141.7988 74.8496) (width 0.127) (layer "F.Cu") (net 3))
 (segment (start 141.7988 74.8496) (end 142.1879 74.4605) (width 0.127) (layer "F.Cu") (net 3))
 (segment (start 142.55 72.6948) (end 142.55 73.6346) (width 0.4) (layer "F.Cu") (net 3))
 (via (at 142.1879 74.354484) (size 0.5) (drill 0.3) (layers "F.Cu" "B.Cu") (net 3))
 (via (at 139.402684 77.2485) (size 0.5) (drill 0.3) (layers "F.Cu" "B.Cu") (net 3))
 (via (at 140.699616 79.206216) (size 0.5) (drill 0.3) (layers "F.Cu" "B.Cu") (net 3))
 (segment (start 139.402684 77.2485) (end 139.402684 77.1397) (width 0.127) (layer "B.Cu") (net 3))
 (segment (start 139.402684 77.1397) (end 142.1879 74.354484) (width 0.127) (layer "B.Cu") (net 3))
 (segment (start 139.402684 77.2485) (end 139.402684 77.909284) (width 0.127) (layer "B.Cu") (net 3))
 (segment (start 139.402684 77.909284) (end 140.699616 79.206216) (width 0.127) (layer "B.Cu") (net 3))
 (segment (start 135.4685 79.1315) (end 135.7096 79.3726) (width 0.4) (layer "F.Cu") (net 5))
 (segment (start 134.65 79.7) (end 135.3435 79.0065) (width 0.4) (layer "F.Cu") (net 5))
 (segment (start 134.9952 78.6582) (end 135.3435 79.0065) (width 0.4) (layer "F.Cu") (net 5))
 (segment (start 135.4685 79.1315) (end 135.4685 79.9685) (width 0.4) (layer "F.Cu") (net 5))
 (segment (start 135.4685 79.9685) (end 135.95 80.45) (width 0.4) (layer "F.Cu") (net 5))
 (segment (start 134.5158 78.6582) (end 134.9952 78.6582) (width 0.4) (layer "F.Cu") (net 5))
 (segment (start 134.65 80.3) (end 134.65 79.7) (width 0.4) (layer "F.Cu") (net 5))
 (segment (start 135.7096 79.3726) (end 135.486 79.3726) (width 0.4) (layer "F.Cu") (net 5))
 (segment (start 134.5158 78.6582) (end 135.6818 78.6582) (width 0.4) (layer "F.Cu") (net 5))
 (segment (start 135.6818 78.6582) (end 135.79 78.55) (width 0.4) (layer "F.Cu") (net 5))
 (segment (start 135.3435 79.0065) (end 135.4685 79.1315) (width 0.4) (layer "F.Cu") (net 5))
 (via (at 134.65 80.3) (size 0.8) (drill 0.4) (layers "F.Cu" "B.Cu") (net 5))
 (segment (start 134.7724 80.0862) (end 134.7724 80.1776) (width 0.4) (layer "B.Cu") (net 5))
 (segment (start 134.7724 79.4766) (end 135.3058 78.9432) (width 0.4) (layer "B.Cu") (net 5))
 (segment (start 134.7724 80.1776) (end 134.65 80.3) (width 0.4) (layer "B.Cu") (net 5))
 (segment (start 134.7724 80.0862) (end 134.7724 79.4766) (width 0.4) (layer "B.Cu") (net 5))
 (segment (start 134.5158 76.39675) (end 134.81255 76.1) (width 0.4) (layer "F.Cu") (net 11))
 (segment (start 134.5158 77.6982) (end 134.5158 76.39675) (width 0.4) (layer "F.Cu") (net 11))
 (segment (start 143.015587 74.438693) (end 142.2988 75.15548) (width 0.25) (layer "F.Cu") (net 6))
 (segment (start 148.4884 76.8146) (end 147.7772 77.5258) (width 0.25) (layer "F.Cu") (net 6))
 (segment (start 148.4884 76.3016) (end 148.4884 76.8146) (width 0.25) (layer "F.Cu") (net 6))
 (segment (start 142.2988 75.15548) (end 142.2988 75.6635) (width 0.25) (layer "F.Cu") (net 6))
 (via (at 148.4884 76.3016) (size 0.5) (drill 0.3) (layers "F.Cu" "B.Cu") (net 6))
 (via (at 143.015587 74.438693) (size 0.5) (drill 0.3) (layers "F.Cu" "B.Cu") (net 6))
 (segment (start 148.276 76.0892) (end 148.4884 76.3016) (width 0.25) (layer "B.Cu") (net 6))
 (segment (start 144.666094 76.0892) (end 148.276 76.0892) (width 0.25) (layer "B.Cu") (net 6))
 (segment (start 143.015587 74.438693) (end 144.666094 76.0892) (width 0.25) (layer "B.Cu") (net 6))
 (segment (start 143.015587 74.438693) (end 143.442507 74.438693) (width 0.25) (layer "B.Cu") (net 6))
 (segment (start 143.442507 74.438693) (end 144.3482 73.533) (width 0.25) (layer "B.Cu") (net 6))
 (segment (start 137.260199 75.139999) (end 138.5018 76.3816) (width 0.4) (layer "F.Cu") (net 4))
 (segment (start 136.398 74.350549) (end 137.18745 75.139999) (width 0.4) (layer "F.Cu") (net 4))
 (segment (start 136.398 73.6092) (end 136.398 74.350549) (width 0.4) (layer "F.Cu") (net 4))
 (segment (start 140.122964 76.851) (end 140.6113 76.851) (width 0.254) (layer "F.Cu") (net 4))
 (segment (start 138.5018 74.1172) (end 138.5018 76.3816) (width 0.4) (layer "F.Cu") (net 4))
 (segment (start 139.550326 76.3816) (end 139.915363 76.746637) (width 0.4) (layer "F.Cu") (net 4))
 (segment (start 139.653564 76.3816) (end 140.122964 76.851) (width 0.254) (layer "F.Cu") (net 4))
 (segment (start 137.18745 75.139999) (end 137.260199 75.139999) (width 0.4) (layer "F.Cu") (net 4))
 (segment (start 138.43 76.3816) (end 139.550326 76.3816) (width 0.4) (layer "F.Cu") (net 4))
 (segment (start 139.0352 73.5838) (end 138.5018 74.1172) (width 0.4) (layer "F.Cu") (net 4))
 (segment (start 138.3494 76.3816) (end 139.653564 76.3816) (width 0.254) (layer "F.Cu") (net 4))
 (segment (start 143.9863 76.851) (end 143.9883 76.853) (width 0.254) (layer "F.Cu") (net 8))
 (segment (start 146.952 75.692) (end 147.6756 75.692) (width 0.4) (layer "F.Cu") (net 8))
 (segment (start 144.8848 76.853) (end 144.9578 76.926) (width 0.254) (layer "F.Cu") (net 8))
 (segment (start 147.057 73.6092) (end 147.057 75.395884) (width 0.4) (layer "F.Cu") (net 8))
 (segment (start 145.526884 76.926) (end 144.9578 76.926) (width 0.4) (layer "F.Cu") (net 8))
 (segment (start 143.9883 76.853) (end 144.8848 76.853) (width 0.254) (layer "F.Cu") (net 8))
 (segment (start 147.6756 75.692) (end 147.8534 75.5142) (width 0.4) (layer "F.Cu") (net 8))
 (segment (start 147.057 75.395884) (end 145.526884 76.926) (width 0.4) (layer "F.Cu") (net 8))
 (via (at 147.8534 75.5142) (size 0.5) (drill 0.3) (layers "F.Cu" "B.Cu") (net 8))
 (segment (start 147.8534 75.5142) (end 147.8534 74.2442) (width 0.4) (layer "B.Cu") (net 8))
 (segment (start 147.8534 74.2442) (end 147.1422 73.533) (width 0.4) (layer "B.Cu") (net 8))
 (segment (start 139.573 77.851) (end 140.6113 77.851) (width 0.25) (layer "F.Cu") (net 12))
 (segment (start 144.0248 77.3895) (end 146.1559 77.3895) (width 0.127) (layer "F.Cu") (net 15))
 (segment (start 143.9863 77.351) (end 144.0248 77.3895) (width 0.127) (layer "F.Cu") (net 15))
 (segment (start 146.1559 77.3895) (end 146.3548 77.1906) (width 0.127) (layer "F.Cu") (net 15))
 (via (at 146.3548 77.1906) (size 0.5) (drill 0.3) (layers "F.Cu" "B.Cu") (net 15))
 (segment (start 146.558 77.3938) (end 147.5994 77.3938) (width 0.127) (layer "B.Cu") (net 15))
 (segment (start 146.3548 77.1906) (end 146.558 77.3938) (width 0.127) (layer "B.Cu") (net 15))
 (segment (start 141.1134 75.5031) (end 141.2738 75.6635) (width 0.4) (layer "F.Cu") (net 16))
 (segment (start 141.1134 73.5838) (end 141.1134 75.5031) (width 0.4) (layer "F.Cu") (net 16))
 (segment (start 144.907 74.7092) (end 143.9527 75.6635) (width 0.4) (layer "F.Cu") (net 7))
 (segment (start 143.9527 75.6635) (end 143.3238 75.6635) (width 0.4) (layer "F.Cu") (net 7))
 (segment (start 144.907 73.6092) (end 144.907 74.7092) (width 0.4) (layer "F.Cu") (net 7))
 (segment (start 142.2988 80.4498) (end 143.0274 81.1784) (width 0.254) (layer "F.Cu") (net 14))
 (segment (start 146.1262 79.0174) (end 146.1516 78.992) (width 0.254) (layer "F.Cu") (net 14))
 (segment (start 143.0274 81.1784) (end 142.3416 81.1784) (width 0.254) (layer "F.Cu") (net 14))
 (segment (start 142.2988 80.4592) (end 142.2988 79.0385) (width 0.254) (layer "F.Cu") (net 14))
 (segment (start 146.1262 80.137) (end 146.1262 79.0174) (width 0.254) (layer "F.Cu") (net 14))
 (segment (start 141.5796 81.1784) (end 142.2988 80.4592) (width 0.254) (layer "F.Cu") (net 14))
 (segment (start 142.3416 81.1784) (end 142.3162 81.2038) (width 0.254) (layer "F.Cu") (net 14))
 (segment (start 142.2988 79.0385) (end 142.2988 80.4498) (width 0.254) (layer "F.Cu") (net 14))
 (via (at 146.1262 80.137) (size 0.8) (drill 0.4) (layers "F.Cu" "B.Cu") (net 14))
 (via (at 142.3162 81.2038) (size 0.8) (drill 0.4) (layers "F.Cu" "B.Cu") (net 14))
 (segment (start 145.0594 81.2038) (end 146.1262 80.137) (width 0.254) (layer "B.Cu") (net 14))
 (segment (start 142.3162 81.2038) (end 145.0594 81.2038) (width 0.254) (layer "B.Cu") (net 14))
 (segment (start 143.9926 80.1624) (end 143.0314 80.1624) (width 0.254) (layer "F.Cu") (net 9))
 (segment (start 143.2988 79.887) (end 143.2988 79.0385) (width 0.254) (layer "F.Cu") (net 9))
 (segment (start 143.0314 80.1624) (end 143.0274 80.1584) (width 0.254) (layer "F.Cu") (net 9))
 (segment (start 143.0274 80.1584) (end 143.2988 79.887) (width 0.254) (layer "F.Cu") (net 9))
 (segment (start 140.6144 80.1604) (end 141.5776 80.1604) (width 0.254) (layer "F.Cu") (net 13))
 (segment (start 141.7988 79.0385) (end 141.7988 79.9392) (width 0.127) (layer "F.Cu") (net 13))
 (segment (start 141.5776 80.1604) (end 141.5796 80.1584) (width 0.254) (layer "F.Cu") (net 13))
 (segment (start 141.7988 79.9392) (end 141.5796 80.1584) (width 0.127) (layer "F.Cu") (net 13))
 (segment (start 143.9863 77.851) (end 144.9558 77.851) (width 0.25) (layer "F.Cu") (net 10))
 (segment (start 145.1316 78.0268) (end 145.1316 78.992) (width 0.25) (layer "F.Cu") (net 10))
 (segment (start 144.9558 77.851) (end 145.1316 78.0268) (width 0.25) (layer "F.Cu") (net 10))
 (segment (start 144.9578 79.8884) (end 143.9863 78.9169) (width 0.254) (layer "F.Cu") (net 1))
 (segment (start 143.9926 81.135766) (end 144.9578 80.170566) (width 0.254) (layer "F.Cu") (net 1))
 (segment (start 143.9863 78.9169) (end 143.9863 78.351) (width 0.254) (layer "F.Cu") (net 1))
 (segment (start 144.9578 80.170566) (end 144.9578 80.1584) (width 0.254) (layer "F.Cu") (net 1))
 (segment (start 144.9578 80.1584) (end 144.9578 79.8884) (width 0.254) (layer "F.Cu") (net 1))
 (segment (start 143.9926 81.1824) (end 143.9926 81.135766) (width 0.254) (layer "F.Cu") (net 1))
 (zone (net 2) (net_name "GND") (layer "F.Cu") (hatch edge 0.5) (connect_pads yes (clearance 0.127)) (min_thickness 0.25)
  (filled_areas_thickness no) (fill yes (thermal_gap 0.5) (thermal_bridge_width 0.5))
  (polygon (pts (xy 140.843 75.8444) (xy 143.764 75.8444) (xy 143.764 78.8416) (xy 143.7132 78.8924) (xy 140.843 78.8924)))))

